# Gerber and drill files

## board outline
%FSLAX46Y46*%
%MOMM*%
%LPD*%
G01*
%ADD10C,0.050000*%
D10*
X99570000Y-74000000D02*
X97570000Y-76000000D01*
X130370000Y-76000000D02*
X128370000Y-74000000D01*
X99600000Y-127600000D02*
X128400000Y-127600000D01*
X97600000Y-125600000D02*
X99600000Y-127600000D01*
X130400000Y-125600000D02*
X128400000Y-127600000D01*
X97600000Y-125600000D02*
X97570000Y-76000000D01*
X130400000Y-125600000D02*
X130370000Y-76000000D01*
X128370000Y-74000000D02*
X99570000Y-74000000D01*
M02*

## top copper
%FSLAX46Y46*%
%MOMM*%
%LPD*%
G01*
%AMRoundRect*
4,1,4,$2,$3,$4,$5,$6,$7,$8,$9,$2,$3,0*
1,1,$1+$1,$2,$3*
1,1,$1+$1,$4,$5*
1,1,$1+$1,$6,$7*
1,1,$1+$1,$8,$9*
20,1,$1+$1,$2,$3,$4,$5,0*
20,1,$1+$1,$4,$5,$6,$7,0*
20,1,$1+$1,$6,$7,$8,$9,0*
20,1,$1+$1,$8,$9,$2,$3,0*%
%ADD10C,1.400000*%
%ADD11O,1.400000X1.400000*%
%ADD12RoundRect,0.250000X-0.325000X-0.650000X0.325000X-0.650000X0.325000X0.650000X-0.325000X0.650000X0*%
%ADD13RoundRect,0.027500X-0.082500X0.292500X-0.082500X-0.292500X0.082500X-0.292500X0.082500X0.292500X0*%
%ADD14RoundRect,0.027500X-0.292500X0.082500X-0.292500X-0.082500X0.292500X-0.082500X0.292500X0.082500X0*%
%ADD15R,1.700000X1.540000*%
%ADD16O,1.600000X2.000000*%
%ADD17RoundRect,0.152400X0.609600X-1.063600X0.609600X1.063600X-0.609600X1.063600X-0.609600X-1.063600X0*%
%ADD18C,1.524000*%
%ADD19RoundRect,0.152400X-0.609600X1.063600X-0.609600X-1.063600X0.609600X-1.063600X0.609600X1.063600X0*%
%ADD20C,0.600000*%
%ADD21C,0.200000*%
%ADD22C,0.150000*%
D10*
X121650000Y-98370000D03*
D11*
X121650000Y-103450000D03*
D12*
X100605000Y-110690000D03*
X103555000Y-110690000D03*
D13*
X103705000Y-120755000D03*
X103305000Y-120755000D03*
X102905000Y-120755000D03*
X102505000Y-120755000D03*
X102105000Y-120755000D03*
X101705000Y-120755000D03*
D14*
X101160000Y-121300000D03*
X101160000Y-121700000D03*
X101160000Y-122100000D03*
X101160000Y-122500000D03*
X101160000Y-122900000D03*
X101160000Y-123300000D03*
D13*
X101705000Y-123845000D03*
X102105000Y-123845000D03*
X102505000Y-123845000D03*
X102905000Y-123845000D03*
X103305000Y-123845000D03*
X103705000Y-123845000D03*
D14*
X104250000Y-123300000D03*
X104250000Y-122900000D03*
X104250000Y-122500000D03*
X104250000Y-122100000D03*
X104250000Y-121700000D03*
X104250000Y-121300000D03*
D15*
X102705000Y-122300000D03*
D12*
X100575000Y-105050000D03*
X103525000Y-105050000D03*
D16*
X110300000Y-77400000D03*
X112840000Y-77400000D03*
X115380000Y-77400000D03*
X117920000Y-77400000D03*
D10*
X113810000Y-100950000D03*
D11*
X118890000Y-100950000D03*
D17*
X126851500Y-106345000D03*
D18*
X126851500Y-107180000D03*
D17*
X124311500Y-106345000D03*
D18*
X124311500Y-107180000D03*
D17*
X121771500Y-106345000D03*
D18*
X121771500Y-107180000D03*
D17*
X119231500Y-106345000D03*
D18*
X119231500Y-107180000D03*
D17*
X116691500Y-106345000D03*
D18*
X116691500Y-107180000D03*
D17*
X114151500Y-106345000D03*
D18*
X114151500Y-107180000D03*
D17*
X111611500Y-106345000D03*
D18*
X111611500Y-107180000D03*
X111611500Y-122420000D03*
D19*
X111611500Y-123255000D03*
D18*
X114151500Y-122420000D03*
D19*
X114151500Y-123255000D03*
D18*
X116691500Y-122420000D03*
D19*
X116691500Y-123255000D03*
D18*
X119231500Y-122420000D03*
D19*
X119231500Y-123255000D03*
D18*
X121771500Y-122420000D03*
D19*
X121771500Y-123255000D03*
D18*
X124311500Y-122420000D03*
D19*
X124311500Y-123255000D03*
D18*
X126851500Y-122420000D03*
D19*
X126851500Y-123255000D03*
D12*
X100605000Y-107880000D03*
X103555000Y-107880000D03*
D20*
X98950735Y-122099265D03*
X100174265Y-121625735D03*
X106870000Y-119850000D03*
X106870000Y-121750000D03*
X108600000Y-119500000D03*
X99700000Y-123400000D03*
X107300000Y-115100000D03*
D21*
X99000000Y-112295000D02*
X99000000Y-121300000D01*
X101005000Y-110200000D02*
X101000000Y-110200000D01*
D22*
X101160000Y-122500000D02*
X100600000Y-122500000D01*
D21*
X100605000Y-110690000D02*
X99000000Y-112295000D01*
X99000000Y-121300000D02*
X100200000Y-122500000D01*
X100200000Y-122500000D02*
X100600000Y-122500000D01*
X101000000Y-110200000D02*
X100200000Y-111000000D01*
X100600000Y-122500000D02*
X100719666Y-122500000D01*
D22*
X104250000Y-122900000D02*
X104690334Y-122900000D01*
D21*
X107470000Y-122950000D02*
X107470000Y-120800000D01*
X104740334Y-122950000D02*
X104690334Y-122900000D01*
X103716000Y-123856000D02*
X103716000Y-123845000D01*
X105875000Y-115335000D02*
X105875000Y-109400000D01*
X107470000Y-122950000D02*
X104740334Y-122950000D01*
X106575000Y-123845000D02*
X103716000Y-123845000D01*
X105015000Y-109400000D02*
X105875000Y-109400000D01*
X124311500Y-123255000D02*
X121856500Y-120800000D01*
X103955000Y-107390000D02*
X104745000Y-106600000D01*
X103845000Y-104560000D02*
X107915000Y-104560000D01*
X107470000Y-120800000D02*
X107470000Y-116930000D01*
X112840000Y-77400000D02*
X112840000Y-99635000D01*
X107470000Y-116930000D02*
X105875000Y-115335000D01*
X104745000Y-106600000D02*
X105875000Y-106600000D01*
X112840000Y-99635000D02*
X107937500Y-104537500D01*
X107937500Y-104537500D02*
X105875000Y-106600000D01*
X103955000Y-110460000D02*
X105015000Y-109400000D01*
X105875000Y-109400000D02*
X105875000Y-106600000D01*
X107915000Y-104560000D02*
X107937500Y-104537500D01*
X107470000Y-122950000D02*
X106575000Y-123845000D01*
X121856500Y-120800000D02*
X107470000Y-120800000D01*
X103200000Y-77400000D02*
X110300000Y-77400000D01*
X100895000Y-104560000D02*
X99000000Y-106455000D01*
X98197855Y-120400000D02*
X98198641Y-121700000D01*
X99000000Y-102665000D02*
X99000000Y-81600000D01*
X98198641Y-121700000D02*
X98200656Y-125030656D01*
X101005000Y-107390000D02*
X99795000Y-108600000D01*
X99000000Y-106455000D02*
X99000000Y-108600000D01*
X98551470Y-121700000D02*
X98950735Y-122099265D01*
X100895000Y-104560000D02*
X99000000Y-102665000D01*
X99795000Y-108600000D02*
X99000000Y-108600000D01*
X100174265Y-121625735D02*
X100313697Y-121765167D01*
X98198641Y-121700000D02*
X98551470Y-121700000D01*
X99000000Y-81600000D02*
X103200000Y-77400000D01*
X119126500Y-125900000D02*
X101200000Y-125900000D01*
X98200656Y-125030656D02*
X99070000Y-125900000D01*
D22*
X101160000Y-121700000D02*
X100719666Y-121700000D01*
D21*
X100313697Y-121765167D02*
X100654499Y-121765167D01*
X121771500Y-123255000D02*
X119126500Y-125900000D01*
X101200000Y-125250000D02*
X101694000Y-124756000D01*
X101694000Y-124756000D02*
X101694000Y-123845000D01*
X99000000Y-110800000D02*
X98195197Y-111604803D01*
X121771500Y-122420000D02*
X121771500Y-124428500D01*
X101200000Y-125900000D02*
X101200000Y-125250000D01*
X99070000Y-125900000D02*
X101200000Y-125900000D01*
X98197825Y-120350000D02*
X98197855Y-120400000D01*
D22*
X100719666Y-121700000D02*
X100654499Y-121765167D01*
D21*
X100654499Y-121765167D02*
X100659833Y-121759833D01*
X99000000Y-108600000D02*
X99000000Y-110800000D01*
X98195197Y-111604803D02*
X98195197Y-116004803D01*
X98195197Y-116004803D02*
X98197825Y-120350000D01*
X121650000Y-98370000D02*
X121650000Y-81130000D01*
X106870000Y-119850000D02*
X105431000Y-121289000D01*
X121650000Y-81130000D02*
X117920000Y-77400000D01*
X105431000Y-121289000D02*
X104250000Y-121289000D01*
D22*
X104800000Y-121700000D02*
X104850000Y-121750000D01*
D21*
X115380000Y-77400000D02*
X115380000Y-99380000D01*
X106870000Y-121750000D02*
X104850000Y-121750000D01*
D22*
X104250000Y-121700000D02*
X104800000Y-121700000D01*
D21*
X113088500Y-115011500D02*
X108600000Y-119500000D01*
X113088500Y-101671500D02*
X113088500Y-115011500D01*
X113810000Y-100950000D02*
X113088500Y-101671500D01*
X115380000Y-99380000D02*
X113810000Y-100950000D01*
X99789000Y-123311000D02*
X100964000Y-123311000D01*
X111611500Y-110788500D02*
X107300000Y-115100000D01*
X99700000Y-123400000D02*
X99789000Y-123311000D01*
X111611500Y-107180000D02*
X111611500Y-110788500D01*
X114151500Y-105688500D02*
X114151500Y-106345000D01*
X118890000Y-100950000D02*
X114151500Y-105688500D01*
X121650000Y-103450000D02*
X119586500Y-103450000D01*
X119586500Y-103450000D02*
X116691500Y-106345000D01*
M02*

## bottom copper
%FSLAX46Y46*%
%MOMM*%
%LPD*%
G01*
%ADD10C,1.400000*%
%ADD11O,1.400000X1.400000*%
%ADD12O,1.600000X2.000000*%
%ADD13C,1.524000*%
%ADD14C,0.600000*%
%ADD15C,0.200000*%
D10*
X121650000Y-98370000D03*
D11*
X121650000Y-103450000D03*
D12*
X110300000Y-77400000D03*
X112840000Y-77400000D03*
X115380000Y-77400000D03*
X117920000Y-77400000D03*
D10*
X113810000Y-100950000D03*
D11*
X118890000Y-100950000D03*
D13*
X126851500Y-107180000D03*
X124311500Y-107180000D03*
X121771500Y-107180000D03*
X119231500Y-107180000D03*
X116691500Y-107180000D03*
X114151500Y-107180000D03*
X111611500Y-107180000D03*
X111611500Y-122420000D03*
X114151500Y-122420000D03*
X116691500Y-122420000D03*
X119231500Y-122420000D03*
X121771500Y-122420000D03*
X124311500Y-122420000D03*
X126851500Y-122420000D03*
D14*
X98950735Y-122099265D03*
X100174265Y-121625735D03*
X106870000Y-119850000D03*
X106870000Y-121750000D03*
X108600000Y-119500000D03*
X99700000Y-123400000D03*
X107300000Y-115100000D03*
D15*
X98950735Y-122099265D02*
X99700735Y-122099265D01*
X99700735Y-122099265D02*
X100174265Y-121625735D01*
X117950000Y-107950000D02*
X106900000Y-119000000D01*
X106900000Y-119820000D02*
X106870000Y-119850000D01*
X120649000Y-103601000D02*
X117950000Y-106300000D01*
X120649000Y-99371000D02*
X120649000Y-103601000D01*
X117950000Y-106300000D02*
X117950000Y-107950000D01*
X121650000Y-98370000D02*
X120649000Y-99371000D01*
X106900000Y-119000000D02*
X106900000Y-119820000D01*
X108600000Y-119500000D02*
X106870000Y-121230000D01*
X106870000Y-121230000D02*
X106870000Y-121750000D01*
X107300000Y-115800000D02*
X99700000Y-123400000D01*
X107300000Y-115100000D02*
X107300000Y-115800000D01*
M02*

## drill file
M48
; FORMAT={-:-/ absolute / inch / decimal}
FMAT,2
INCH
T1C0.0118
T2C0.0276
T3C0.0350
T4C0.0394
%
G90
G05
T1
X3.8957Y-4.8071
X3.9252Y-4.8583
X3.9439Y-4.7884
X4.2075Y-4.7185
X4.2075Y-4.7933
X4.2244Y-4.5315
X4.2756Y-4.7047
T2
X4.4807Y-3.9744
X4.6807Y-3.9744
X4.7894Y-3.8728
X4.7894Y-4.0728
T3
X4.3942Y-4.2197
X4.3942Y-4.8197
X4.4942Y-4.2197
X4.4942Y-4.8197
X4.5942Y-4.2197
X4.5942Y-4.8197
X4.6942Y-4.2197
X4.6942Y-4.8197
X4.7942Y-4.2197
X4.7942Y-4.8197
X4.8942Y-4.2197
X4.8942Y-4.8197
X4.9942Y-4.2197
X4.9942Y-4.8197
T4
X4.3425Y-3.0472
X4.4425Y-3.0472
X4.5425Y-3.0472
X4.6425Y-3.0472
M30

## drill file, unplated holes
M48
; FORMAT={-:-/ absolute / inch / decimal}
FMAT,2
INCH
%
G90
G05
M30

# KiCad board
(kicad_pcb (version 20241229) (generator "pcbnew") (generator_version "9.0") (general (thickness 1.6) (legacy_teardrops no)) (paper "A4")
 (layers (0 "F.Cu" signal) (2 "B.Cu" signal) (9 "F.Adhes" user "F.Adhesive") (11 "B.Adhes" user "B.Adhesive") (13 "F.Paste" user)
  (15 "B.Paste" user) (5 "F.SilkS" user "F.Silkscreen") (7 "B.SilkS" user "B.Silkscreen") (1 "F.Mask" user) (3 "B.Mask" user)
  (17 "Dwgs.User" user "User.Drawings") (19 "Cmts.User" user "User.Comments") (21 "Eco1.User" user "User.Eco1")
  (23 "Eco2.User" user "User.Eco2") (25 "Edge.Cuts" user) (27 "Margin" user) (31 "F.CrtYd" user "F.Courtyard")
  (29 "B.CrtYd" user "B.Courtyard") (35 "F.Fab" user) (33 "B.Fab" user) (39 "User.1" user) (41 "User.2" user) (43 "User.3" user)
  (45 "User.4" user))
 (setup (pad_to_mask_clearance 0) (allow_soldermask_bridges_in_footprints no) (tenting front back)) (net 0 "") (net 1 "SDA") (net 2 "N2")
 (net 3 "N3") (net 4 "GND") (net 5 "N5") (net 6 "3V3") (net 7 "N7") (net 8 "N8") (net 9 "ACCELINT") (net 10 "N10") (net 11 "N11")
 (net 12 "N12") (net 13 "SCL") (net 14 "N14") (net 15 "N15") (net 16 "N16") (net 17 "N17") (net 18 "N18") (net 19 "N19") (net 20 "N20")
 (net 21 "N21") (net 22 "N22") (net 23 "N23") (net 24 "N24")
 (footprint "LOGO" (layer "F.Cu") (at 127.4 126)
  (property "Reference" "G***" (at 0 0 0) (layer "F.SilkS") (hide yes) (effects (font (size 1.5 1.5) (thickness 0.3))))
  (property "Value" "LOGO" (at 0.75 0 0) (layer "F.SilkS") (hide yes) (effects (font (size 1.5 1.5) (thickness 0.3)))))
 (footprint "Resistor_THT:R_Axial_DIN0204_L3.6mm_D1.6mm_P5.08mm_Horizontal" (layer "F.Cu") (at 121.65 98.37 -90)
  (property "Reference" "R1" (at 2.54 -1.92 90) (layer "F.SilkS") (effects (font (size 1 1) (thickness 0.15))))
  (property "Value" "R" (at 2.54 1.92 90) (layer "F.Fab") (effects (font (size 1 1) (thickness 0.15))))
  (pad "1" thru_hole circle (at 0 0 270) (size 1.4 1.4) (drill 0.7) (layers "*.Cu" "*.Mask") (remove_unused_layers no) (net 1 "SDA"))
  (pad "2" thru_hole oval (at 5.08 0 270) (size 1.4 1.4) (drill 0.7) (layers "*.Cu" "*.Mask") (remove_unused_layers no) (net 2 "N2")))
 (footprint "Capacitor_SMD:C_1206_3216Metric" (layer "F.Cu") (at 102.08 110.69)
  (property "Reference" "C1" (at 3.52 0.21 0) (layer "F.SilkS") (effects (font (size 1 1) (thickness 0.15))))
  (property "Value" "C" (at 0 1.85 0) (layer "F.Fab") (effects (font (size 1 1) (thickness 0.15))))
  (pad "1" smd roundrect (at -1.475 0) (size 1.15 1.8) (layers "F.Cu" "F.Mask" "F.Paste") (roundrect_rratio 0.217391) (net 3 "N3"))
  (pad "2" smd roundrect (at 1.475 0) (size 1.15 1.8) (layers "F.Cu" "F.Mask" "F.Paste") (roundrect_rratio 0.217391) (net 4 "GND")))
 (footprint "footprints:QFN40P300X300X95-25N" (layer "F.Cu") (at 102.705 122.3 -90)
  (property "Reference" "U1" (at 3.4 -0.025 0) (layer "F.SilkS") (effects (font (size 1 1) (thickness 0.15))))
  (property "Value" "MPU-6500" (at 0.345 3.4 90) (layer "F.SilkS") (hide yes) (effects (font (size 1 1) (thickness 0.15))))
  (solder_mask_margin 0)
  (pad "1" smd roundrect (at -1.545 -1 270) (size 0.64 0.22) (layers "F.Cu" "F.Mask" "F.Paste") (roundrect_rratio 0.125)
   (solder_mask_margin 0.102))
  (pad "2" smd roundrect (at -1.545 -0.6 270) (size 0.64 0.22) (layers "F.Cu" "F.Mask" "F.Paste") (roundrect_rratio 0.125)
   (solder_mask_margin 0.102))
  (pad "3" smd roundrect (at -1.545 -0.2 270) (size 0.64 0.22) (layers "F.Cu" "F.Mask" "F.Paste") (roundrect_rratio 0.125)
   (solder_mask_margin 0.102))
  (pad "4" smd roundrect (at -1.545 0.2 270) (size 0.64 0.22) (layers "F.Cu" "F.Mask" "F.Paste") (roundrect_rratio 0.125)
   (solder_mask_margin 0.102))
  (pad "5" smd roundrect (at -1.545 0.6 270) (size 0.64 0.22) (layers "F.Cu" "F.Mask" "F.Paste") (roundrect_rratio 0.125)
   (solder_mask_margin 0.102))
  (pad "6" smd roundrect (at -1.545 1 270) (size 0.64 0.22) (layers "F.Cu" "F.Mask" "F.Paste") (roundrect_rratio 0.125)
   (solder_mask_margin 0.102))
  (pad "7" smd roundrect (at -1 1.545 270) (size 0.22 0.64) (layers "F.Cu" "F.Mask" "F.Paste") (roundrect_rratio 0.125) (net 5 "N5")
   (solder_mask_margin 0.102))
  (pad "8" smd roundrect (at -0.6 1.545 270) (size 0.22 0.64) (layers "F.Cu" "F.Mask" "F.Paste") (roundrect_rratio 0.125) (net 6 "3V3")
   (solder_mask_margin 0.102))
  (pad "9" smd roundrect (at -0.2 1.545 270) (size 0.22 0.64) (layers "F.Cu" "F.Mask" "F.Paste") (roundrect_rratio 0.125) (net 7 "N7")
   (solder_mask_margin 0.102))
  (pad "10" smd roundrect (at 0.2 1.545 270) (size 0.22 0.64) (layers "F.Cu" "F.Mask" "F.Paste") (roundrect_rratio 0.125) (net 3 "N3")
   (solder_mask_margin 0.102))
  (pad "11" smd roundrect (at 0.6 1.545 270) (size 0.22 0.64) (layers "F.Cu" "F.Mask" "F.Paste") (roundrect_rratio 0.125) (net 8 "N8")
   (solder_mask_margin 0.102))
  (pad "12" smd roundrect (at 1 1.545 270) (size 0.22 0.64) (layers "F.Cu" "F.Mask" "F.Paste") (roundrect_rratio 0.125) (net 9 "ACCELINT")
   (solder_mask_margin 0.102))
  (pad "13" smd roundrect (at 1.545 1 270) (size 0.64 0.22) (layers "F.Cu" "F.Mask" "F.Paste") (roundrect_rratio 0.125) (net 6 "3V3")
   (solder_mask_margin 0.102))
  (pad "14" smd roundrect (at 1.545 0.6 270) (size 0.64 0.22) (layers "F.Cu" "F.Mask" "F.Paste") (roundrect_rratio 0.125)
   (solder_mask_margin 0.102))
  (pad "15" smd roundrect (at 1.545 0.2 270) (size 0.64 0.22) (layers "F.Cu" "F.Mask" "F.Paste") (roundrect_rratio 0.125)
   (solder_mask_margin 0.102))
  (pad "16" smd roundrect (at 1.545 -0.2 270) (size 0.64 0.22) (layers "F.Cu" "F.Mask" "F.Paste") (roundrect_rratio 0.125)
   (solder_mask_margin 0.102))
  (pad "17" smd roundrect (at 1.545 -0.6 270) (size 0.64 0.22) (layers "F.Cu" "F.Mask" "F.Paste") (roundrect_rratio 0.125)
   (solder_mask_margin 0.102))
  (pad "18" smd roundrect (at 1.545 -1 270) (size 0.64 0.22) (layers "F.Cu" "F.Mask" "F.Paste") (roundrect_rratio 0.125) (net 4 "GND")
   (solder_mask_margin 0.102))
  (pad "19" smd roundrect (at 1 -1.545 270) (size 0.22 0.64) (layers "F.Cu" "F.Mask" "F.Paste") (roundrect_rratio 0.125) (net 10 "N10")
   (solder_mask_margin 0.102))
  (pad "20" smd roundrect (at 0.6 -1.545 270) (size 0.22 0.64) (layers "F.Cu" "F.Mask" "F.Paste") (roundrect_rratio 0.125) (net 4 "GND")
   (solder_mask_margin 0.102))
  (pad "21" smd roundrect (at 0.2 -1.545 270) (size 0.22 0.64) (layers "F.Cu" "F.Mask" "F.Paste") (roundrect_rratio 0.125) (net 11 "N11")
   (solder_mask_margin 0.102))
  (pad "22" smd roundrect (at -0.2 -1.545 270) (size 0.22 0.64) (layers "F.Cu" "F.Mask" "F.Paste") (roundrect_rratio 0.125) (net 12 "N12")
   (solder_mask_margin 0.102))
  (pad "23" smd roundrect (at -0.6 -1.545 270) (size 0.22 0.64) (layers "F.Cu" "F.Mask" "F.Paste") (roundrect_rratio 0.125) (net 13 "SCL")
   (solder_mask_margin 0.102))
  (pad "24" smd roundrect (at -1 -1.545 270) (size 0.22 0.64) (layers "F.Cu" "F.Mask" "F.Paste") (roundrect_rratio 0.125) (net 1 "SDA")
   (solder_mask_margin 0.102))
  (pad "25" smd rect (at 0 0 270) (size 1.54 1.7) (layers "F.Cu" "F.Mask") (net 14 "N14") (solder_mask_margin 0.102)))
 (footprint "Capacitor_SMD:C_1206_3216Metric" (layer "F.Cu") (at 102.05 105.05)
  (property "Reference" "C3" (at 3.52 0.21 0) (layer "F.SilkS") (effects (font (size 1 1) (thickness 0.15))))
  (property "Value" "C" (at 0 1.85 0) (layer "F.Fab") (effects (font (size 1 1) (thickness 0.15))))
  (pad "1" smd roundrect (at -1.475 0) (size 1.15 1.8) (layers "F.Cu" "F.Mask" "F.Paste") (roundrect_rratio 0.217391) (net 6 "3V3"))
  (pad "2" smd roundrect (at 1.475 0) (size 1.15 1.8) (layers "F.Cu" "F.Mask" "F.Paste") (roundrect_rratio 0.217391) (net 4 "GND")))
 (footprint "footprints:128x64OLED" (layer "F.Cu") (at 113.92 88)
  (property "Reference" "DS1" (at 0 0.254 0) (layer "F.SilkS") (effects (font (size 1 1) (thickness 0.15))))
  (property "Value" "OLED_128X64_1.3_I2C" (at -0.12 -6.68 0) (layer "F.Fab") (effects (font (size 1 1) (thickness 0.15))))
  (pad "1" thru_hole oval (at -3.62 -10.6 90) (size 2 1.6) (drill 1) (layers "*.Cu" "*.Mask") (remove_unused_layers no) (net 6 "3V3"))
  (pad "2" thru_hole oval (at -1.08 -10.6 90) (size 2 1.6) (drill 1) (layers "*.Cu" "*.Mask") (remove_unused_layers no) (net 4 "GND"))
  (pad "3" thru_hole oval (at 1.46 -10.6 90) (size 2 1.6) (drill 1) (layers "*.Cu" "*.Mask") (remove_unused_layers no) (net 13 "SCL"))
  (pad "4" thru_hole oval (at 4 -10.6 90) (size 2 1.6) (drill 1) (layers "*.Cu" "*.Mask") (remove_unused_layers no) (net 1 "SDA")))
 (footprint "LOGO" (layer "F.Cu") (at 102.6 116.6)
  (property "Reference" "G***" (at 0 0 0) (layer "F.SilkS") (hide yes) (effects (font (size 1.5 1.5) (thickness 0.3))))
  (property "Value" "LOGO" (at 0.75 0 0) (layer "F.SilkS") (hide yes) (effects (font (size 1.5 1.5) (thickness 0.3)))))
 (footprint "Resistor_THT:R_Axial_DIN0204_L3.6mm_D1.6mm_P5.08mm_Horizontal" (layer "F.Cu") (at 113.81 100.95)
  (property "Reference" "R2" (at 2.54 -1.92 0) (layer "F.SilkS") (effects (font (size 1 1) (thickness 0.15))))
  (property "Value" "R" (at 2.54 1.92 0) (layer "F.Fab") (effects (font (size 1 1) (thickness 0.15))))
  (pad "1" thru_hole circle (at 0 0) (size 1.4 1.4) (drill 0.7) (layers "*.Cu" "*.Mask") (remove_unused_layers no) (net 13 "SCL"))
  (pad "2" thru_hole oval (at 5.08 0) (size 1.4 1.4) (drill 0.7) (layers "*.Cu" "*.Mask") (remove_unused_layers no) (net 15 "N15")))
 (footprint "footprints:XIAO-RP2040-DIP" (layer "F.Cu") (at 119.2315 114.8 -90)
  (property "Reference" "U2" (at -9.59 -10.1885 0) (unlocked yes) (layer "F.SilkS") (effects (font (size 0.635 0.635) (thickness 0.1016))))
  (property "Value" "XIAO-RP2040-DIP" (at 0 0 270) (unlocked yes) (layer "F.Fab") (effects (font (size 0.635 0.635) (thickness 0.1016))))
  (pad "1" smd roundrect (at -8.455 -7.62 90) (size 2.432 1.524) (layers "F.Cu" "F.Mask") (roundrect_rratio 0.1) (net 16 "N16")
   (thermal_bridge_angle 45))
  (pad "1" thru_hole circle (at -7.62 -7.62 90) (size 1.524 1.524) (drill 0.889) (layers "*.Cu" "*.Mask") (remove_unused_layers no)
   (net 16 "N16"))
  (pad "2" smd roundrect (at -8.455 -5.08 90) (size 2.432 1.524) (layers "F.Cu" "F.Mask") (roundrect_rratio 0.1) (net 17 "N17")
   (thermal_bridge_angle 45))
  (pad "2" thru_hole circle (at -7.62 -5.08 90) (size 1.524 1.524) (drill 0.889) (layers "*.Cu" "*.Mask") (remove_unused_layers no)
   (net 17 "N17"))
  (pad "3" smd roundrect (at -8.455 -2.54 90) (size 2.432 1.524) (layers "F.Cu" "F.Mask") (roundrect_rratio 0.1) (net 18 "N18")
   (thermal_bridge_angle 45))
  (pad "3" thru_hole circle (at -7.62 -2.54 90) (size 1.524 1.524) (drill 0.889) (layers "*.Cu" "*.Mask") (remove_unused_layers no)
   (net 18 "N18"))
  (pad "4" smd roundrect (at -8.455 0 90) (size 2.432 1.524) (layers "F.Cu" "F.Mask") (roundrect_rratio 0.1) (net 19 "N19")
   (thermal_bridge_angle 45))
  (pad "4" thru_hole circle (at -7.62 0 90) (size 1.524 1.524) (drill 0.889) (layers "*.Cu" "*.Mask") (remove_unused_layers no)
   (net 19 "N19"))
  (pad "5" smd roundrect (at -8.455 2.54 90) (size 2.432 1.524) (layers "F.Cu" "F.Mask") (roundrect_rratio 0.1) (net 2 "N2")
   (thermal_bridge_angle 45))
  (pad "5" thru_hole circle (at -7.62 2.54 90) (size 1.524 1.524) (drill 0.889) (layers "*.Cu" "*.Mask") (remove_unused_layers no)
   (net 2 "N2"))
  (pad "6" smd roundrect (at -8.455 5.08 90) (size 2.432 1.524) (layers "F.Cu" "F.Mask") (roundrect_rratio 0.1) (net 15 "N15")
   (thermal_bridge_angle 45))
  (pad "6" thru_hole circle (at -7.62 5.08 90) (size 1.524 1.524) (drill 0.889) (layers "*.Cu" "*.Mask") (remove_unused_layers no)
   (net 15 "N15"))
  (pad "7" smd roundrect (at -8.455 7.62 90) (size 2.432 1.524) (layers "F.Cu" "F.Mask") (roundrect_rratio 0.1) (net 9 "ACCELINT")
   (thermal_bridge_angle 45))
  (pad "7" thru_hole circle (at -7.62 7.62 90) (size 1.524 1.524) (drill 0.889) (layers "*.Cu" "*.Mask") (remove_unused_layers no)
   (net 9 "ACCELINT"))
  (pad "8" thru_hole circle (at 7.62 7.62 270) (size 1.524 1.524) (drill 0.889) (layers "*.Cu" "*.Mask") (remove_unused_layers no)
   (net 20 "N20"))
  (pad "8" smd roundrect (at 8.455 7.62 270) (size 2.432 1.524) (layers "F.Cu" "F.Mask") (roundrect_rratio 0.1) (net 20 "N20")
   (thermal_bridge_angle 45))
  (pad "9" thru_hole circle (at 7.62 5.08 270) (size 1.524 1.524) (drill 0.889) (layers "*.Cu" "*.Mask") (remove_unused_layers no)
   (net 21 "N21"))
  (pad "9" smd roundrect (at 8.455 5.08 270) (size 2.432 1.524) (layers "F.Cu" "F.Mask") (roundrect_rratio 0.1) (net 21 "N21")
   (thermal_bridge_angle 45))
  (pad "10" thru_hole circle (at 7.62 2.54 270) (size 1.524 1.524) (drill 0.889) (layers "*.Cu" "*.Mask") (remove_unused_layers no)
   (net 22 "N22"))
  (pad "10" smd roundrect (at 8.455 2.54 270) (size 2.432 1.524) (layers "F.Cu" "F.Mask") (roundrect_rratio 0.1) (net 22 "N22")
   (thermal_bridge_angle 45))
  (pad "11" thru_hole circle (at 7.62 0 270) (size 1.524 1.524) (drill 0.889) (layers "*.Cu" "*.Mask") (remove_unused_layers no)
   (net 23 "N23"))
  (pad "11" smd roundrect (at 8.455 0 270) (size 2.432 1.524) (layers "F.Cu" "F.Mask") (roundrect_rratio 0.1) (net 23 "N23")
   (thermal_bridge_angle 45))
  (pad "12" thru_hole circle (at 7.62 -2.54 270) (size 1.524 1.524) (drill 0.889) (layers "*.Cu" "*.Mask") (remove_unused_layers no)
   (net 6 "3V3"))
  (pad "12" smd roundrect (at 8.455 -2.54 270) (size 2.432 1.524) (layers "F.Cu" "F.Mask") (roundrect_rratio 0.1) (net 6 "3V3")
   (thermal_bridge_angle 45))
  (pad "13" thru_hole circle (at 7.62 -5.08 270) (size 1.524 1.524) (drill 0.889) (layers "*.Cu" "*.Mask") (remove_unused_layers no)
   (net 4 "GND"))
  (pad "13" smd roundrect (at 8.455 -5.08 270) (size 2.432 1.524) (layers "F.Cu" "F.Mask") (roundrect_rratio 0.1) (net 4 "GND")
   (thermal_bridge_angle 45))
  (pad "14" thru_hole circle (at 7.62 -7.62 270) (size 1.524 1.524) (drill 0.889) (layers "*.Cu" "*.Mask") (remove_unused_layers no)
   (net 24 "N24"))
  (pad "14" smd roundrect (at 8.455 -7.62 270) (size 2.432 1.524) (layers "F.Cu" "F.Mask") (roundrect_rratio 0.1) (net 24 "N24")
   (thermal_bridge_angle 45)))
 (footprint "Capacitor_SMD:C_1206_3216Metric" (layer "F.Cu") (at 102.08 107.88)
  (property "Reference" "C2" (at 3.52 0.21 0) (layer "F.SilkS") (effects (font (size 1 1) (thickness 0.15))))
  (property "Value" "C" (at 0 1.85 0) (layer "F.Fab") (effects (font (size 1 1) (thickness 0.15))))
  (pad "1" smd roundrect (at -1.475 0) (size 1.15 1.8) (layers "F.Cu" "F.Mask" "F.Paste") (roundrect_rratio 0.217391) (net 6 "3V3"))
  (pad "2" smd roundrect (at 1.475 0) (size 1.15 1.8) (layers "F.Cu" "F.Mask" "F.Paste") (roundrect_rratio 0.217391) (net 4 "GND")))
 (gr_line (start 99.57 74) (end 97.57 76) (stroke (width 0.05) (type default)) (layer "Edge.Cuts"))
 (gr_line (start 130.37 76) (end 128.37 74) (stroke (width 0.05) (type default)) (layer "Edge.Cuts"))
 (gr_line (start 99.6 127.6) (end 128.4 127.6) (stroke (width 0.05) (type default)) (layer "Edge.Cuts"))
 (gr_line (start 97.6 125.6) (end 99.6 127.6) (stroke (width 0.05) (type default)) (layer "Edge.Cuts"))
 (gr_line (start 130.4 125.6) (end 128.4 127.6) (stroke (width 0.05) (type default)) (layer "Edge.Cuts"))
 (gr_line (start 97.6 125.6) (end 97.57 76) (stroke (width 0.05) (type default)) (layer "Edge.Cuts"))
 (gr_line (start 130.4 125.6) (end 130.37 76) (stroke (width 0.05) (type default)) (layer "Edge.Cuts"))
 (gr_line (start 128.37 74) (end 99.57 74) (stroke (width 0.05) (type default)) (layer "Edge.Cuts"))
 (segment (start 99 112.295) (end 99 121.3) (width 0.2) (layer "F.Cu") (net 3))
 (segment (start 101.005 110.2) (end 101 110.2) (width 0.2) (layer "F.Cu") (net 3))
 (segment (start 101.16 122.5) (end 100.6 122.5) (width 0.15) (layer "F.Cu") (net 3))
 (segment (start 100.605 110.69) (end 99 112.295) (width 0.2) (layer "F.Cu") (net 3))
 (segment (start 99 121.3) (end 100.2 122.5) (width 0.2) (layer "F.Cu") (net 3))
 (segment (start 100.2 122.5) (end 100.6 122.5) (width 0.2) (layer "F.Cu") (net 3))
 (segment (start 101 110.2) (end 100.2 111) (width 0.2) (layer "F.Cu") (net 3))
 (segment (start 100.6 122.5) (end 100.719666 122.5) (width 0.2) (layer "F.Cu") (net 3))
 (segment (start 104.25 122.9) (end 104.690334 122.9) (width 0.15) (layer "F.Cu") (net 4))
 (segment (start 107.47 122.95) (end 107.47 120.8) (width 0.2) (layer "F.Cu") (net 4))
 (segment (start 104.740334 122.95) (end 104.690334 122.9) (width 0.2) (layer "F.Cu") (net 4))
 (segment (start 103.716 123.856) (end 103.716 123.845) (width 0.2) (layer "F.Cu") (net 4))
 (segment (start 105.875 115.335) (end 105.875 109.4) (width 0.2) (layer "F.Cu") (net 4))
 (segment (start 107.47 122.95) (end 104.740334 122.95) (width 0.2) (layer "F.Cu") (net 4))
 (segment (start 106.575 123.845) (end 103.716 123.845) (width 0.2) (layer "F.Cu") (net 4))
 (segment (start 105.015 109.4) (end 105.875 109.4) (width 0.2) (layer "F.Cu") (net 4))
 (segment (start 124.3115 123.255) (end 121.8565 120.8) (width 0.2) (layer "F.Cu") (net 4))
 (segment (start 103.955 107.39) (end 104.745 106.6) (width 0.2) (layer "F.Cu") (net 4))
 (segment (start 103.845 104.56) (end 107.915 104.56) (width 0.2) (layer "F.Cu") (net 4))
 (segment (start 107.47 120.8) (end 107.47 116.93) (width 0.2) (layer "F.Cu") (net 4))
 (segment (start 112.84 77.4) (end 112.84 99.635) (width 0.2) (layer "F.Cu") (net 4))
 (segment (start 107.47 116.93) (end 105.875 115.335) (width 0.2) (layer "F.Cu") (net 4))
 (segment (start 104.745 106.6) (end 105.875 106.6) (width 0.2) (layer "F.Cu") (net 4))
 (segment (start 112.84 99.635) (end 107.9375 104.5375) (width 0.2) (layer "F.Cu") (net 4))
 (segment (start 107.9375 104.5375) (end 105.875 106.6) (width 0.2) (layer "F.Cu") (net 4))
 (segment (start 103.955 110.46) (end 105.015 109.4) (width 0.2) (layer "F.Cu") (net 4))
 (segment (start 105.875 109.4) (end 105.875 106.6) (width 0.2) (layer "F.Cu") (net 4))
 (segment (start 107.915 104.56) (end 107.9375 104.5375) (width 0.2) (layer "F.Cu") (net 4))
 (segment (start 107.47 122.95) (end 106.575 123.845) (width 0.2) (layer "F.Cu") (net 4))
 (segment (start 121.8565 120.8) (end 107.47 120.8) (width 0.2) (layer "F.Cu") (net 4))
 (segment (start 103.2 77.4) (end 110.3 77.4) (width 0.2) (layer "F.Cu") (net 6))
 (segment (start 100.895 104.56) (end 99 106.455) (width 0.2) (layer "F.Cu") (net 6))
 (segment (start 98.197855 120.4) (end 98.198641 121.7) (width 0.2) (layer "F.Cu") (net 6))
 (segment (start 99 102.665) (end 99 81.6) (width 0.2) (layer "F.Cu") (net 6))
 (segment (start 98.198641 121.7) (end 98.200656 125.030656) (width 0.2) (layer "F.Cu") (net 6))
 (segment (start 101.005 107.39) (end 99.795 108.6) (width 0.2) (layer "F.Cu") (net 6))
 (segment (start 99 106.455) (end 99 108.6) (width 0.2) (layer "F.Cu") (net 6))
 (segment (start 98.55147 121.7) (end 98.950735 122.099265) (width 0.2) (layer "F.Cu") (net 6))
 (segment (start 100.895 104.56) (end 99 102.665) (width 0.2) (layer "F.Cu") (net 6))
 (segment (start 99.795 108.6) (end 99 108.6) (width 0.2) (layer "F.Cu") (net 6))
 (segment (start 100.174265 121.625735) (end 100.313697 121.765167) (width 0.2) (layer "F.Cu") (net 6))
 (segment (start 98.198641 121.7) (end 98.55147 121.7) (width 0.2) (layer "F.Cu") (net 6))
 (segment (start 99 81.6) (end 103.2 77.4) (width 0.2) (layer "F.Cu") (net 6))
 (segment (start 119.1265 125.9) (end 101.2 125.9) (width 0.2) (layer "F.Cu") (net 6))
 (segment (start 98.200656 125.030656) (end 99.07 125.9) (width 0.2) (layer "F.Cu") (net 6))
 (segment (start 101.16 121.7) (end 100.719666 121.7) (width 0.15) (layer "F.Cu") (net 6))
 (segment (start 100.313697 121.765167) (end 100.654499 121.765167) (width 0.2) (layer "F.Cu") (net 6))
 (segment (start 121.7715 123.255) (end 119.1265 125.9) (width 0.2) (layer "F.Cu") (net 6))
 (segment (start 101.2 125.25) (end 101.694 124.756) (width 0.2) (layer "F.Cu") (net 6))
 (segment (start 101.694 124.756) (end 101.694 123.845) (width 0.2) (layer "F.Cu") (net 6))
 (segment (start 99 110.8) (end 98.195197 111.604803) (width 0.2) (layer "F.Cu") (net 6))
 (segment (start 121.7715 122.42) (end 121.7715 124.4285) (width 0.2) (layer "F.Cu") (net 6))
 (segment (start 101.2 125.9) (end 101.2 125.25) (width 0.2) (layer "F.Cu") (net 6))
 (segment (start 99.07 125.9) (end 101.2 125.9) (width 0.2) (layer "F.Cu") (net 6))
 (segment (start 98.197825 120.35) (end 98.197855 120.4) (width 0.2) (layer "F.Cu") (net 6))
 (segment (start 100.719666 121.7) (end 100.654499 121.765167) (width 0.15) (layer "F.Cu") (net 6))
 (segment (start 100.654499 121.765167) (end 100.659833 121.759833) (width 0.2) (layer "F.Cu") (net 6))
 (segment (start 99 108.6) (end 99 110.8) (width 0.2) (layer "F.Cu") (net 6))
 (segment (start 98.195197 111.604803) (end 98.195197 116.004803) (width 0.2) (layer "F.Cu") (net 6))
 (segment (start 98.195197 116.004803) (end 98.197825 120.35) (width 0.2) (layer "F.Cu") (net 6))
 (via (at 98.950735 122.099265) (size 0.6) (drill 0.3) (layers "F.Cu" "B.Cu") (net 6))
 (via (at 100.174265 121.625735) (size 0.6) (drill 0.3) (layers "F.Cu" "B.Cu") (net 6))
 (segment (start 98.950735 122.099265) (end 99.700735 122.099265) (width 0.2) (layer "B.Cu") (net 6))
 (segment (start 99.700735 122.099265) (end 100.174265 121.625735) (width 0.2) (layer "B.Cu") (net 6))
 (segment (start 121.65 98.37) (end 121.65 81.13) (width 0.2) (layer "F.Cu") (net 1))
 (segment (start 106.87 119.85) (end 105.431 121.289) (width 0.2) (layer "F.Cu") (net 1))
 (segment (start 121.65 81.13) (end 117.92 77.4) (width 0.2) (layer "F.Cu") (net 1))
 (segment (start 105.431 121.289) (end 104.25 121.289) (width 0.2) (layer "F.Cu") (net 1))
 (via (at 106.87 119.85) (size 0.6) (drill 0.3) (layers "F.Cu" "B.Cu") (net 1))
 (segment (start 117.95 107.95) (end 106.9 119) (width 0.2) (layer "B.Cu") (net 1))
 (segment (start 106.9 119.82) (end 106.87 119.85) (width 0.2) (layer "B.Cu") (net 1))
 (segment (start 120.649 103.601) (end 117.95 106.3) (width 0.2) (layer "B.Cu") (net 1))
 (segment (start 120.649 99.371) (end 120.649 103.601) (width 0.2) (layer "B.Cu") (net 1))
 (segment (start 117.95 106.3) (end 117.95 107.95) (width 0.2) (layer "B.Cu") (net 1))
 (segment (start 121.65 98.37) (end 120.649 99.371) (width 0.2) (layer "B.Cu") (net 1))
 (segment (start 106.9 119) (end 106.9 119.82) (width 0.2) (layer "B.Cu") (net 1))
 (segment (start 104.8 121.7) (end 104.85 121.75) (width 0.15) (layer "F.Cu") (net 13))
 (segment (start 115.38 77.4) (end 115.38 99.38) (width 0.2) (layer "F.Cu") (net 13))
 (segment (start 106.87 121.75) (end 104.85 121.75) (width 0.2) (layer "F.Cu") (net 13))
 (segment (start 104.25 121.7) (end 104.8 121.7) (width 0.15) (layer "F.Cu") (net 13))
 (segment (start 113.0885 115.0115) (end 108.6 119.5) (width 0.2) (layer "F.Cu") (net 13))
 (segment (start 113.0885 101.6715) (end 113.0885 115.0115) (width 0.2) (layer "F.Cu") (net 13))
 (segment (start 113.81 100.95) (end 113.0885 101.6715) (width 0.2) (layer "F.Cu") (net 13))
 (segment (start 115.38 99.38) (end 113.81 100.95) (width 0.2) (layer "F.Cu") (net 13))
 (via (at 106.87 121.75) (size 0.6) (drill 0.3) (layers "F.Cu" "B.Cu") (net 13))
 (via (at 108.6 119.5) (size 0.6) (drill 0.3) (layers "F.Cu" "B.Cu") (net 13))
 (segment (start 108.6 119.5) (end 106.87 121.23) (width 0.2) (layer "B.Cu") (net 13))
 (segment (start 106.87 121.23) (end 106.87 121.75) (width 0.2) (layer "B.Cu") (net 13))
 (segment (start 99.789 123.311) (end 100.964 123.311) (width 0.2) (layer "F.Cu") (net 9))
 (segment (start 111.6115 110.7885) (end 107.3 115.1) (width 0.2) (layer "F.Cu") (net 9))
 (segment (start 99.7 123.4) (end 99.789 123.311) (width 0.2) (layer "F.Cu") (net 9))
 (segment (start 111.6115 107.18) (end 111.6115 110.7885) (width 0.2) (layer "F.Cu") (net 9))
 (via (at 99.7 123.4) (size 0.6) (drill 0.3) (layers "F.Cu" "B.Cu") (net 9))
 (via (at 107.3 115.1) (size 0.6) (drill 0.3) (layers "F.Cu" "B.Cu") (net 9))
 (segment (start 107.3 115.8) (end 99.7 123.4) (width 0.2) (layer "B.Cu") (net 9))
 (segment (start 107.3 115.1) (end 107.3 115.8) (width 0.2) (layer "B.Cu") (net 9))
 (segment (start 114.1515 105.6885) (end 114.1515 106.345) (width 0.2) (layer "F.Cu") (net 15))
 (segment (start 118.89 100.95) (end 114.1515 105.6885) (width 0.2) (layer "F.Cu") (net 15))
 (segment (start 121.65 103.45) (end 119.5865 103.45) (width 0.2) (layer "F.Cu") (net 2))
 (segment (start 119.5865 103.45) (end 116.6915 106.345) (width 0.2) (layer "F.Cu") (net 2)))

